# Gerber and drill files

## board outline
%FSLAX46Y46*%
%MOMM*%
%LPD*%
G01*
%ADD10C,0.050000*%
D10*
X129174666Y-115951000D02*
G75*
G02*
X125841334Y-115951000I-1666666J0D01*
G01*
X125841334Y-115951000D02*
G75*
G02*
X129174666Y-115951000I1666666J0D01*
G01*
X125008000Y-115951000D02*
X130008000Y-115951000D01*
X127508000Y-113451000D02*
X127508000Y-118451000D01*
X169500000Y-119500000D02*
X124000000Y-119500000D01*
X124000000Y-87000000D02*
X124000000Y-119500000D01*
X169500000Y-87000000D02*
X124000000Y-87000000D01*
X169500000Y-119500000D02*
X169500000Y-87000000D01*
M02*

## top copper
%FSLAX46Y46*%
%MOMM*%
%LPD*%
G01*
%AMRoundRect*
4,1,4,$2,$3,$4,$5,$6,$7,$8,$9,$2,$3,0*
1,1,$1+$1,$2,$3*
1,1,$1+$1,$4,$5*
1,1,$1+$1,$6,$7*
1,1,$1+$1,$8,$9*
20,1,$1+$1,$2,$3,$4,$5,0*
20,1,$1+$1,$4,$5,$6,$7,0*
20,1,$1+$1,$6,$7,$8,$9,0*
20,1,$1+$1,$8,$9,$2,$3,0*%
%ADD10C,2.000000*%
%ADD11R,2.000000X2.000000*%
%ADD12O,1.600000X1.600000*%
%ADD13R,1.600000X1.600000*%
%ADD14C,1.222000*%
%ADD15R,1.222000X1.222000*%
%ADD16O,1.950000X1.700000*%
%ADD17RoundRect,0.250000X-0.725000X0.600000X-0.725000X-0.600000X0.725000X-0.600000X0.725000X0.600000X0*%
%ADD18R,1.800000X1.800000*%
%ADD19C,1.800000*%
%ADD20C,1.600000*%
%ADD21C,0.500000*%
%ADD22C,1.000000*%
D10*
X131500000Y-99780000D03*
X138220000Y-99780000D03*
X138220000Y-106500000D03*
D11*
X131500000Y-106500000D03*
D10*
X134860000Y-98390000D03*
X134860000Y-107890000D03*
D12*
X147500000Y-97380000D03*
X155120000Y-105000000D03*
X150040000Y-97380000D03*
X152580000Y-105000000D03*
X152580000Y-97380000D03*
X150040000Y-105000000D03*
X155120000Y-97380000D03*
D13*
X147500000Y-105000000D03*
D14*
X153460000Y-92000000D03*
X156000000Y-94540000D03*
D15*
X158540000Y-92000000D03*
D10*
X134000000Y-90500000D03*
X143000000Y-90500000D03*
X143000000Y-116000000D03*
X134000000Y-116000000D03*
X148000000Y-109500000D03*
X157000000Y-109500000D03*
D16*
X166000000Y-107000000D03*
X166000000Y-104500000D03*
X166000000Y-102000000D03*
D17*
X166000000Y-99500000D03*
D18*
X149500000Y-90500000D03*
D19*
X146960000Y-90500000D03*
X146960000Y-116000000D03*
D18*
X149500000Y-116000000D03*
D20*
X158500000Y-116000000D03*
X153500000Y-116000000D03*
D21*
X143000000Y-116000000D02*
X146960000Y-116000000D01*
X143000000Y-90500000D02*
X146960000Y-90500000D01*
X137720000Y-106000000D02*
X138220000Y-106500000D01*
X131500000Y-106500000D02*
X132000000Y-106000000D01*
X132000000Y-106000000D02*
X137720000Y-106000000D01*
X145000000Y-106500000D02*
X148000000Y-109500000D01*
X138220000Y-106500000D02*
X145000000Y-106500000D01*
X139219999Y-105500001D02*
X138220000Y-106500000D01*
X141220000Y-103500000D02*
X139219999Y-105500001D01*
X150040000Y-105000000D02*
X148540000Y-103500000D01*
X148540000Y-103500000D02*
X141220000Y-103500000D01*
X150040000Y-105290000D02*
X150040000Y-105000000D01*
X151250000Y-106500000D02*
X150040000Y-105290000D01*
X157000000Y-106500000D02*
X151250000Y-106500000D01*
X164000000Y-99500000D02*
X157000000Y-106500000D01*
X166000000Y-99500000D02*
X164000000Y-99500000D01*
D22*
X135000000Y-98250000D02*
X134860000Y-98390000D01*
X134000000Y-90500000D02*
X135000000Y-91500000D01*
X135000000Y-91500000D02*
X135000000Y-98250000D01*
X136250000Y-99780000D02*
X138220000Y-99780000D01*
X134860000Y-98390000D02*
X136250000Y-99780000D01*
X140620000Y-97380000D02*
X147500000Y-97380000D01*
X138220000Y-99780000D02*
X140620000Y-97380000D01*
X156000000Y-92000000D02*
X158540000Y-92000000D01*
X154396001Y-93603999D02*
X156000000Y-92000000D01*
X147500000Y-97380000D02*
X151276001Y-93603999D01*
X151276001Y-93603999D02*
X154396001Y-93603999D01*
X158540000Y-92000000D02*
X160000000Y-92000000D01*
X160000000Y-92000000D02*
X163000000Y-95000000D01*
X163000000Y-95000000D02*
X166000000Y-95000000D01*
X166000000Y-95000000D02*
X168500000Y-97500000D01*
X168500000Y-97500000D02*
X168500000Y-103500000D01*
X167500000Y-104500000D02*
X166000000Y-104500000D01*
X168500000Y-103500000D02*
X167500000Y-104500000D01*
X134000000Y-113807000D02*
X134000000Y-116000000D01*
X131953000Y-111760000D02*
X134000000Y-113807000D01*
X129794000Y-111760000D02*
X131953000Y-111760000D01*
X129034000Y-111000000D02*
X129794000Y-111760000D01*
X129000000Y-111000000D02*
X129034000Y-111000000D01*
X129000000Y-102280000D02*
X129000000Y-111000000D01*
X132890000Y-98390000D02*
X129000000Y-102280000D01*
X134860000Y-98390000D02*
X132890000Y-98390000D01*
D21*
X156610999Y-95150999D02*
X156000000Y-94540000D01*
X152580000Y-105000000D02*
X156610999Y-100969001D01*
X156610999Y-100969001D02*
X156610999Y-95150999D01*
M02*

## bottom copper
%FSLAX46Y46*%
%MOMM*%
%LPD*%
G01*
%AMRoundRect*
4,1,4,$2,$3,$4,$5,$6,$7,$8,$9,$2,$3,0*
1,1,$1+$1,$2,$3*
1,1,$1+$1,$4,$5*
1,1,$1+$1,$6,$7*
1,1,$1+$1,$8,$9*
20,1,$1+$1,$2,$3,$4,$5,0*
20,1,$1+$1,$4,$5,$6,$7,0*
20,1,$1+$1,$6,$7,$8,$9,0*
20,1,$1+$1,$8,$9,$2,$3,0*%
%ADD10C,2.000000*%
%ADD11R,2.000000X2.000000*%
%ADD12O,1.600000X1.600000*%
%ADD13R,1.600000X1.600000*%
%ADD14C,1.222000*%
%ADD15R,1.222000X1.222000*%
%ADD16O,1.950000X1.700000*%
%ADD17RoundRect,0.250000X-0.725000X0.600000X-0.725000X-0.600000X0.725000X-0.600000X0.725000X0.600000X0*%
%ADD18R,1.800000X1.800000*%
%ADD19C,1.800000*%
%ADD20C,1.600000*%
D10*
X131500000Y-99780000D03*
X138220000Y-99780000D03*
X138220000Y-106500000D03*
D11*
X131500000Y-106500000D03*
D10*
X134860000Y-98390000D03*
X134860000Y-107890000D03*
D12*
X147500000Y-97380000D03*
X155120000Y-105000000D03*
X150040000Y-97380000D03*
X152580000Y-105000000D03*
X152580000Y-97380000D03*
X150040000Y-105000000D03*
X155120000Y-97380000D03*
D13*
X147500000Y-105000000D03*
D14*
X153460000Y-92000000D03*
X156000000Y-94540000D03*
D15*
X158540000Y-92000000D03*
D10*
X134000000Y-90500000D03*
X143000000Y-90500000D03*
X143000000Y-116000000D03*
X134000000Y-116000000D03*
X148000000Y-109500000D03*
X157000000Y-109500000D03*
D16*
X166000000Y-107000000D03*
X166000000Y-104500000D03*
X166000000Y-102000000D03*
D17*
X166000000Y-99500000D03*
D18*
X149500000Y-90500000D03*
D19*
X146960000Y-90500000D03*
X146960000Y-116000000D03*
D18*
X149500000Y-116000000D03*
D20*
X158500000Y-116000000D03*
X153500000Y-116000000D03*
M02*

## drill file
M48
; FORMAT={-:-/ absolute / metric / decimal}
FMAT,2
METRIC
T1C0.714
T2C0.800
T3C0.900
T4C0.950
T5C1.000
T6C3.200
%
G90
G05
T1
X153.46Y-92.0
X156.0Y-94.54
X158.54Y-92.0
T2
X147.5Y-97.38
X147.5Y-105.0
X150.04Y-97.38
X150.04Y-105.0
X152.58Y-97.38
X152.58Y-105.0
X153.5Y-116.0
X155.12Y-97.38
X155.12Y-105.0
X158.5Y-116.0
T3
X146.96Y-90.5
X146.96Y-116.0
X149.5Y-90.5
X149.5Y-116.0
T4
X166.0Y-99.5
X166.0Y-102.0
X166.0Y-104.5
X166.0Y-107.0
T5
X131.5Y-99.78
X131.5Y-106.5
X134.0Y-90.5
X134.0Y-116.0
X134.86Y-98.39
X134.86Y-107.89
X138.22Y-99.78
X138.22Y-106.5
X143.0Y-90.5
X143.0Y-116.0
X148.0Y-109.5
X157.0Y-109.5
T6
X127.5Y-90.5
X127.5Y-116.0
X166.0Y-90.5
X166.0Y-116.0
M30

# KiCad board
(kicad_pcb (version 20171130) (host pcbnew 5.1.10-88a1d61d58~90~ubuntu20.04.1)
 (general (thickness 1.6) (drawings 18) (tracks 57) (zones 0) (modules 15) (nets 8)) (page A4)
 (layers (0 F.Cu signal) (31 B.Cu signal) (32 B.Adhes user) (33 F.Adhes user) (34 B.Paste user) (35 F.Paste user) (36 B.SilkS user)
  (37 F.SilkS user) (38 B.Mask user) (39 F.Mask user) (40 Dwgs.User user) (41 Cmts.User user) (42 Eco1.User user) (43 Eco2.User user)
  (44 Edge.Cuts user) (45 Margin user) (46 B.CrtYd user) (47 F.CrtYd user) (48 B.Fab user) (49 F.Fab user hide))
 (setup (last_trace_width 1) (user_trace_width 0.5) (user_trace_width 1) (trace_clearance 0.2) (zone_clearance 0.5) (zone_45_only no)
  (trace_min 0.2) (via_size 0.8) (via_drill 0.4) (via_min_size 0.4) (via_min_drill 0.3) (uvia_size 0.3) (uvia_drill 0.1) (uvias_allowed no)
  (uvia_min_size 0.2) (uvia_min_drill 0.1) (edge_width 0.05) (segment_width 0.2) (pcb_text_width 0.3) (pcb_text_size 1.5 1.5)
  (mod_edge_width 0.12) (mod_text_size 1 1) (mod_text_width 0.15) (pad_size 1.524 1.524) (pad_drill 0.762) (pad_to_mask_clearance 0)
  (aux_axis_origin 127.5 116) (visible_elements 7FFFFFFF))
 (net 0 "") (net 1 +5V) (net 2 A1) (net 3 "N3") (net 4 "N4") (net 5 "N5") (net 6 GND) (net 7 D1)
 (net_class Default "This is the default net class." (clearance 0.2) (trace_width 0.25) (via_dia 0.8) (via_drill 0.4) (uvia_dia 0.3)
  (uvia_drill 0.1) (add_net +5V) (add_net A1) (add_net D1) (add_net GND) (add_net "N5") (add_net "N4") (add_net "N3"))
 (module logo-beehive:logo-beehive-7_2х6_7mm (layer F.Cu) (at 161 113.5 90)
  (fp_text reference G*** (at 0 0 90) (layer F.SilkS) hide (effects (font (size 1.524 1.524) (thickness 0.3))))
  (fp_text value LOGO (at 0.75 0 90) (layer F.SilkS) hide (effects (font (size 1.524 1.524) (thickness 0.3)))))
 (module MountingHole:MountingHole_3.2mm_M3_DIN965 (layer F.Cu) (at 166 90.5)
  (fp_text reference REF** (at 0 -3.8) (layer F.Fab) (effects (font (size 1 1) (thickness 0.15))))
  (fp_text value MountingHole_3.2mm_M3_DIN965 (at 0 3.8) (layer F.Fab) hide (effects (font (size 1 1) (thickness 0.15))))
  (pad 1 np_thru_hole circle (at 0 0) (size 3.2 3.2) (drill 3.2) (layers *.Cu *.Mask)))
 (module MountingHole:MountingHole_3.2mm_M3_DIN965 (layer F.Cu) (at 166 116)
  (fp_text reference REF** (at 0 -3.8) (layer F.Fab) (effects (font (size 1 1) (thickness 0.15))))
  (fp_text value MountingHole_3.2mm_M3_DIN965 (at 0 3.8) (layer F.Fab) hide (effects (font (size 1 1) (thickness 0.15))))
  (pad 1 np_thru_hole circle (at 0 0) (size 3.2 3.2) (drill 3.2) (layers *.Cu *.Mask)))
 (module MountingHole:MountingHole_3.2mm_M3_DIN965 (layer F.Cu) (at 127.5 90.5)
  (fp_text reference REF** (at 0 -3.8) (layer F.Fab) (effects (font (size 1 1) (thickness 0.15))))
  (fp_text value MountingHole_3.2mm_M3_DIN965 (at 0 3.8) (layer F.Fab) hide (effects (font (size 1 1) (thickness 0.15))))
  (pad 1 np_thru_hole circle (at 0 0) (size 3.2 3.2) (drill 3.2) (layers *.Cu *.Mask)))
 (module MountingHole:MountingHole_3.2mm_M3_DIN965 (layer F.Cu) (at 127.5 116)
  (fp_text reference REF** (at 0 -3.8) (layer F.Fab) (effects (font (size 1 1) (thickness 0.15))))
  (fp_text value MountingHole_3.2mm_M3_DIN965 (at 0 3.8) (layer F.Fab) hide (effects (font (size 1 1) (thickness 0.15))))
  (pad 1 np_thru_hole circle (at 0 0) (size 3.2 3.2) (drill 3.2) (layers *.Cu *.Mask)))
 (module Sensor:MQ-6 (layer F.Cu) (at 131.5 106.5 90)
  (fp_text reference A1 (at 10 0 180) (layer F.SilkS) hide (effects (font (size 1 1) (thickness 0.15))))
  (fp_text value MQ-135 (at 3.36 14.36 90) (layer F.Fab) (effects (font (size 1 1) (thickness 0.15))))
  (pad 6 thru_hole circle (at 6.72 0) (size 2 2) (drill 1) (layers *.Cu *.Mask))
  (pad 4 thru_hole circle (at 6.72 6.72 270) (size 2 2) (drill 1) (layers *.Cu *.Mask) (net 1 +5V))
  (pad 3 thru_hole circle (at 0 6.72 180) (size 2 2) (drill 1) (layers *.Cu *.Mask) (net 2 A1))
  (pad 1 thru_hole rect (at 0 0 90) (size 2 2) (drill 1) (layers *.Cu *.Mask) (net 2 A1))
  (pad 5 thru_hole circle (at 8.11 3.36 90) (size 2 2) (drill 1) (layers *.Cu *.Mask) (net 1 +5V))
  (pad 2 thru_hole circle (at -1.39 3.36 90) (size 2 2) (drill 1) (layers *.Cu *.Mask)))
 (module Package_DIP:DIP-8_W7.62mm (layer F.Cu) (at 147.5 105 90)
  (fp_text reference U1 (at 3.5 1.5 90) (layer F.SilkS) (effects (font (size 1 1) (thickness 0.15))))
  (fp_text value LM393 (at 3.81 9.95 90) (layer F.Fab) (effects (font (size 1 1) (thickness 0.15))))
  (pad 8 thru_hole oval (at 7.62 0 90) (size 1.6 1.6) (drill 0.8) (layers *.Cu *.Mask) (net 1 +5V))
  (pad 4 thru_hole oval (at 0 7.62 90) (size 1.6 1.6) (drill 0.8) (layers *.Cu *.Mask))
  (pad 7 thru_hole oval (at 7.62 2.54 90) (size 1.6 1.6) (drill 0.8) (layers *.Cu *.Mask))
  (pad 3 thru_hole oval (at 0 5.08 90) (size 1.6 1.6) (drill 0.8) (layers *.Cu *.Mask) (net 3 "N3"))
  (pad 6 thru_hole oval (at 7.62 5.08 90) (size 1.6 1.6) (drill 0.8) (layers *.Cu *.Mask))
  (pad 2 thru_hole oval (at 0 2.54 90) (size 1.6 1.6) (drill 0.8) (layers *.Cu *.Mask) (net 2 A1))
  (pad 5 thru_hole oval (at 7.62 7.62 90) (size 1.6 1.6) (drill 0.8) (layers *.Cu *.Mask))
  (pad 1 thru_hole rect (at 0 0 90) (size 1.6 1.6) (drill 0.8) (layers *.Cu *.Mask)))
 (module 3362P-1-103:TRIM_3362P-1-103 (layer F.Cu) (at 156 92 180)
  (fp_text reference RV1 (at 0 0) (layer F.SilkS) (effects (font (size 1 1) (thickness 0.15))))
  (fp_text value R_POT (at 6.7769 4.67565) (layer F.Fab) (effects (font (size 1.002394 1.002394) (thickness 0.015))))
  (pad 3 thru_hole circle (at 2.54 0 180) (size 1.222 1.222) (drill 0.714) (layers *.Cu *.Mask))
  (pad 2 thru_hole circle (at 0 -2.54 180) (size 1.222 1.222) (drill 0.714) (layers *.Cu *.Mask) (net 3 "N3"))
  (pad 1 thru_hole rect (at -2.54 0 180) (size 1.222 1.222) (drill 0.714) (layers *.Cu *.Mask) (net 1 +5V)))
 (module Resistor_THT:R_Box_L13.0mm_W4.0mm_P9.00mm (layer F.Cu) (at 134 90.5)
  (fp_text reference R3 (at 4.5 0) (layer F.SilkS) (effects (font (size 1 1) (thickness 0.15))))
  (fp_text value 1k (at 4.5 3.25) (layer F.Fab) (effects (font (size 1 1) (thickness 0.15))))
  (pad 1 thru_hole circle (at 0 0) (size 2 2) (drill 1) (layers *.Cu *.Mask) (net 1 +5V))
  (pad 2 thru_hole circle (at 9 0) (size 2 2) (drill 1) (layers *.Cu *.Mask) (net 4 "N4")))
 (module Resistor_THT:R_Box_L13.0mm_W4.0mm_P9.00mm (layer F.Cu) (at 134 116)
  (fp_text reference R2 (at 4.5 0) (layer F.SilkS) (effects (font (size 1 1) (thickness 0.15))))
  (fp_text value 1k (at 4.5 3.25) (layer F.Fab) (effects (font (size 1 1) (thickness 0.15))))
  (pad 2 thru_hole circle (at 9 0) (size 2 2) (drill 1) (layers *.Cu *.Mask) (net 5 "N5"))
  (pad 1 thru_hole circle (at 0 0) (size 2 2) (drill 1) (layers *.Cu *.Mask) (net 1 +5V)))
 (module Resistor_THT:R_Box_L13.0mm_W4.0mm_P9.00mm (layer F.Cu) (at 148 109.5)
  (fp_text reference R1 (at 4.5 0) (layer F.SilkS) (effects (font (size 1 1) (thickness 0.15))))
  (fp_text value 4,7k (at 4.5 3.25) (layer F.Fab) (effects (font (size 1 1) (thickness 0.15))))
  (pad 1 thru_hole circle (at 0 0) (size 2 2) (drill 1) (layers *.Cu *.Mask) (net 2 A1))
  (pad 2 thru_hole circle (at 9 0) (size 2 2) (drill 1) (layers *.Cu *.Mask)))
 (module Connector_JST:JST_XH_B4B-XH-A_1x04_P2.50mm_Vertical (layer F.Cu) (at 166 99.5 270)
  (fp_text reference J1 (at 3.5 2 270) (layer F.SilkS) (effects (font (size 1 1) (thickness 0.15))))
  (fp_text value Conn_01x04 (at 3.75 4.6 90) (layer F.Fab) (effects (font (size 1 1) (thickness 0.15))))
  (pad 4 thru_hole oval (at 7.5 0 270) (size 1.7 1.95) (drill 0.95) (layers *.Cu *.Mask))
  (pad 3 thru_hole oval (at 5 0 270) (size 1.7 1.95) (drill 0.95) (layers *.Cu *.Mask) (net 1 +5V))
  (pad 2 thru_hole oval (at 2.5 0 270) (size 1.7 1.95) (drill 0.95) (layers *.Cu *.Mask))
  (pad 1 thru_hole roundrect (at 0 0 270) (size 1.7 1.95) (drill 0.95) (layers *.Cu *.Mask) (roundrect_rratio 0.1470588235294118) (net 2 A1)))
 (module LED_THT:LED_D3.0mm (layer F.Cu) (at 149.5 90.5 180)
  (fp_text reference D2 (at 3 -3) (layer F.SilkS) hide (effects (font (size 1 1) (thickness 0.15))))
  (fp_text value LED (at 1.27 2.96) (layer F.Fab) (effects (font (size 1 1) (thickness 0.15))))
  (pad 1 thru_hole rect (at 0 0 180) (size 1.8 1.8) (drill 0.9) (layers *.Cu *.Mask))
  (pad 2 thru_hole circle (at 2.54 0 180) (size 1.8 1.8) (drill 0.9) (layers *.Cu *.Mask) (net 4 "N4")))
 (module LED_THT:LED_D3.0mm (layer F.Cu) (at 149.5 116 180)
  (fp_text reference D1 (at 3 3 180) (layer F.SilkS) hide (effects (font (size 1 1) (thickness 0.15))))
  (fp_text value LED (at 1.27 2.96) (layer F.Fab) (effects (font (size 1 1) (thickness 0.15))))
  (pad 2 thru_hole circle (at 2.54 0 180) (size 1.8 1.8) (drill 0.9) (layers *.Cu *.Mask) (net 5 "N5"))
  (pad 1 thru_hole rect (at 0 0 180) (size 1.8 1.8) (drill 0.9) (layers *.Cu *.Mask)))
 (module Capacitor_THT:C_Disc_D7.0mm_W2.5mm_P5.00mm (layer F.Cu) (at 153.5 116)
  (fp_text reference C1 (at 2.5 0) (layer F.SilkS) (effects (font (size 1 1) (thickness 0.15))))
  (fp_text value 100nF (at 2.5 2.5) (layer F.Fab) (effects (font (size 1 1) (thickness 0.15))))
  (pad 2 thru_hole circle (at 5 0) (size 1.6 1.6) (drill 0.8) (layers *.Cu *.Mask))
  (pad 1 thru_hole circle (at 0 0) (size 1.6 1.6) (drill 0.8) (layers *.Cu *.Mask)))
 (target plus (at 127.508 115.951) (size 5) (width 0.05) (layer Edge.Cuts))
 (gr_line (start 169.5 119.5) (end 124 119.5) (layer Edge.Cuts) (width 0.05))
 (gr_line (start 124 87) (end 124 119.5) (layer Edge.Cuts) (width 0.05))
 (gr_line (start 169.5 87) (end 124 87) (layer Edge.Cuts) (width 0.05))
 (gr_line (start 169.5 119.5) (end 169.5 87) (layer Edge.Cuts) (width 0.05))
 (segment (start 143 116) (end 146.96 116) (width 0.5) (layer F.Cu) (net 5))
 (segment (start 143 90.5) (end 146.96 90.5) (width 0.5) (layer F.Cu) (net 4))
 (segment (start 137.72 106) (end 138.22 106.5) (width 0.5) (layer F.Cu) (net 2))
 (segment (start 131.5 106.5) (end 132 106) (width 0.5) (layer F.Cu) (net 2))
 (segment (start 132 106) (end 137.72 106) (width 0.5) (layer F.Cu) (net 2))
 (segment (start 145 106.5) (end 148 109.5) (width 0.5) (layer F.Cu) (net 2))
 (segment (start 138.22 106.5) (end 145 106.5) (width 0.5) (layer F.Cu) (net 2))
 (segment (start 139.219999 105.500001) (end 138.22 106.5) (width 0.5) (layer F.Cu) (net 2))
 (segment (start 141.22 103.5) (end 139.219999 105.500001) (width 0.5) (layer F.Cu) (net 2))
 (segment (start 150.04 105) (end 148.54 103.5) (width 0.5) (layer F.Cu) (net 2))
 (segment (start 148.54 103.5) (end 141.22 103.5) (width 0.5) (layer F.Cu) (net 2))
 (segment (start 150.04 105.29) (end 150.04 105) (width 0.5) (layer F.Cu) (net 2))
 (segment (start 151.25 106.5) (end 150.04 105.29) (width 0.5) (layer F.Cu) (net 2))
 (segment (start 157 106.5) (end 151.25 106.5) (width 0.5) (layer F.Cu) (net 2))
 (segment (start 164 99.5) (end 157 106.5) (width 0.5) (layer F.Cu) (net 2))
 (segment (start 166 99.5) (end 164 99.5) (width 0.5) (layer F.Cu) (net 2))
 (segment (start 135 98.25) (end 134.86 98.39) (width 1) (layer F.Cu) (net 1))
 (segment (start 134 90.5) (end 135 91.5) (width 1) (layer F.Cu) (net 1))
 (segment (start 135 91.5) (end 135 98.25) (width 1) (layer F.Cu) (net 1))
 (segment (start 136.25 99.78) (end 138.22 99.78) (width 1) (layer F.Cu) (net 1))
 (segment (start 134.86 98.39) (end 136.25 99.78) (width 1) (layer F.Cu) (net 1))
 (segment (start 140.62 97.38) (end 147.5 97.38) (width 1) (layer F.Cu) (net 1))
 (segment (start 138.22 99.78) (end 140.62 97.38) (width 1) (layer F.Cu) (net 1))
 (segment (start 156 92) (end 158.54 92) (width 1) (layer F.Cu) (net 1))
 (segment (start 154.396001 93.603999) (end 156 92) (width 1) (layer F.Cu) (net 1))
 (segment (start 147.5 97.38) (end 151.276001 93.603999) (width 1) (layer F.Cu) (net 1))
 (segment (start 151.276001 93.603999) (end 154.396001 93.603999) (width 1) (layer F.Cu) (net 1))
 (segment (start 158.54 92) (end 160 92) (width 1) (layer F.Cu) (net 1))
 (segment (start 160 92) (end 163 95) (width 1) (layer F.Cu) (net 1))
 (segment (start 163 95) (end 166 95) (width 1) (layer F.Cu) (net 1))
 (segment (start 166 95) (end 168.5 97.5) (width 1) (layer F.Cu) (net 1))
 (segment (start 168.5 97.5) (end 168.5 103.5) (width 1) (layer F.Cu) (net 1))
 (segment (start 167.5 104.5) (end 166 104.5) (width 1) (layer F.Cu) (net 1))
 (segment (start 168.5 103.5) (end 167.5 104.5) (width 1) (layer F.Cu) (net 1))
 (segment (start 134 113.807) (end 134 116) (width 1) (layer F.Cu) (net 1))
 (segment (start 131.953 111.76) (end 134 113.807) (width 1) (layer F.Cu) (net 1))
 (segment (start 129.794 111.76) (end 131.953 111.76) (width 1) (layer F.Cu) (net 1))
 (segment (start 129.034 111) (end 129.794 111.76) (width 1) (layer F.Cu) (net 1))
 (segment (start 129 111) (end 129.034 111) (width 1) (layer F.Cu) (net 1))
 (segment (start 129 102.28) (end 129 111) (width 1) (layer F.Cu) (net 1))
 (segment (start 132.89 98.39) (end 129 102.28) (width 1) (layer F.Cu) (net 1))
 (segment (start 134.86 98.39) (end 132.89 98.39) (width 1) (layer F.Cu) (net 1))
 (segment (start 156.610999 95.150999) (end 156 94.54) (width 0.5) (layer F.Cu) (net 3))
 (segment (start 152.58 105) (end 156.610999 100.969001) (width 0.5) (layer F.Cu) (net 3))
 (segment (start 156.610999 100.969001) (end 156.610999 95.150999) (width 0.5) (layer F.Cu) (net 3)))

